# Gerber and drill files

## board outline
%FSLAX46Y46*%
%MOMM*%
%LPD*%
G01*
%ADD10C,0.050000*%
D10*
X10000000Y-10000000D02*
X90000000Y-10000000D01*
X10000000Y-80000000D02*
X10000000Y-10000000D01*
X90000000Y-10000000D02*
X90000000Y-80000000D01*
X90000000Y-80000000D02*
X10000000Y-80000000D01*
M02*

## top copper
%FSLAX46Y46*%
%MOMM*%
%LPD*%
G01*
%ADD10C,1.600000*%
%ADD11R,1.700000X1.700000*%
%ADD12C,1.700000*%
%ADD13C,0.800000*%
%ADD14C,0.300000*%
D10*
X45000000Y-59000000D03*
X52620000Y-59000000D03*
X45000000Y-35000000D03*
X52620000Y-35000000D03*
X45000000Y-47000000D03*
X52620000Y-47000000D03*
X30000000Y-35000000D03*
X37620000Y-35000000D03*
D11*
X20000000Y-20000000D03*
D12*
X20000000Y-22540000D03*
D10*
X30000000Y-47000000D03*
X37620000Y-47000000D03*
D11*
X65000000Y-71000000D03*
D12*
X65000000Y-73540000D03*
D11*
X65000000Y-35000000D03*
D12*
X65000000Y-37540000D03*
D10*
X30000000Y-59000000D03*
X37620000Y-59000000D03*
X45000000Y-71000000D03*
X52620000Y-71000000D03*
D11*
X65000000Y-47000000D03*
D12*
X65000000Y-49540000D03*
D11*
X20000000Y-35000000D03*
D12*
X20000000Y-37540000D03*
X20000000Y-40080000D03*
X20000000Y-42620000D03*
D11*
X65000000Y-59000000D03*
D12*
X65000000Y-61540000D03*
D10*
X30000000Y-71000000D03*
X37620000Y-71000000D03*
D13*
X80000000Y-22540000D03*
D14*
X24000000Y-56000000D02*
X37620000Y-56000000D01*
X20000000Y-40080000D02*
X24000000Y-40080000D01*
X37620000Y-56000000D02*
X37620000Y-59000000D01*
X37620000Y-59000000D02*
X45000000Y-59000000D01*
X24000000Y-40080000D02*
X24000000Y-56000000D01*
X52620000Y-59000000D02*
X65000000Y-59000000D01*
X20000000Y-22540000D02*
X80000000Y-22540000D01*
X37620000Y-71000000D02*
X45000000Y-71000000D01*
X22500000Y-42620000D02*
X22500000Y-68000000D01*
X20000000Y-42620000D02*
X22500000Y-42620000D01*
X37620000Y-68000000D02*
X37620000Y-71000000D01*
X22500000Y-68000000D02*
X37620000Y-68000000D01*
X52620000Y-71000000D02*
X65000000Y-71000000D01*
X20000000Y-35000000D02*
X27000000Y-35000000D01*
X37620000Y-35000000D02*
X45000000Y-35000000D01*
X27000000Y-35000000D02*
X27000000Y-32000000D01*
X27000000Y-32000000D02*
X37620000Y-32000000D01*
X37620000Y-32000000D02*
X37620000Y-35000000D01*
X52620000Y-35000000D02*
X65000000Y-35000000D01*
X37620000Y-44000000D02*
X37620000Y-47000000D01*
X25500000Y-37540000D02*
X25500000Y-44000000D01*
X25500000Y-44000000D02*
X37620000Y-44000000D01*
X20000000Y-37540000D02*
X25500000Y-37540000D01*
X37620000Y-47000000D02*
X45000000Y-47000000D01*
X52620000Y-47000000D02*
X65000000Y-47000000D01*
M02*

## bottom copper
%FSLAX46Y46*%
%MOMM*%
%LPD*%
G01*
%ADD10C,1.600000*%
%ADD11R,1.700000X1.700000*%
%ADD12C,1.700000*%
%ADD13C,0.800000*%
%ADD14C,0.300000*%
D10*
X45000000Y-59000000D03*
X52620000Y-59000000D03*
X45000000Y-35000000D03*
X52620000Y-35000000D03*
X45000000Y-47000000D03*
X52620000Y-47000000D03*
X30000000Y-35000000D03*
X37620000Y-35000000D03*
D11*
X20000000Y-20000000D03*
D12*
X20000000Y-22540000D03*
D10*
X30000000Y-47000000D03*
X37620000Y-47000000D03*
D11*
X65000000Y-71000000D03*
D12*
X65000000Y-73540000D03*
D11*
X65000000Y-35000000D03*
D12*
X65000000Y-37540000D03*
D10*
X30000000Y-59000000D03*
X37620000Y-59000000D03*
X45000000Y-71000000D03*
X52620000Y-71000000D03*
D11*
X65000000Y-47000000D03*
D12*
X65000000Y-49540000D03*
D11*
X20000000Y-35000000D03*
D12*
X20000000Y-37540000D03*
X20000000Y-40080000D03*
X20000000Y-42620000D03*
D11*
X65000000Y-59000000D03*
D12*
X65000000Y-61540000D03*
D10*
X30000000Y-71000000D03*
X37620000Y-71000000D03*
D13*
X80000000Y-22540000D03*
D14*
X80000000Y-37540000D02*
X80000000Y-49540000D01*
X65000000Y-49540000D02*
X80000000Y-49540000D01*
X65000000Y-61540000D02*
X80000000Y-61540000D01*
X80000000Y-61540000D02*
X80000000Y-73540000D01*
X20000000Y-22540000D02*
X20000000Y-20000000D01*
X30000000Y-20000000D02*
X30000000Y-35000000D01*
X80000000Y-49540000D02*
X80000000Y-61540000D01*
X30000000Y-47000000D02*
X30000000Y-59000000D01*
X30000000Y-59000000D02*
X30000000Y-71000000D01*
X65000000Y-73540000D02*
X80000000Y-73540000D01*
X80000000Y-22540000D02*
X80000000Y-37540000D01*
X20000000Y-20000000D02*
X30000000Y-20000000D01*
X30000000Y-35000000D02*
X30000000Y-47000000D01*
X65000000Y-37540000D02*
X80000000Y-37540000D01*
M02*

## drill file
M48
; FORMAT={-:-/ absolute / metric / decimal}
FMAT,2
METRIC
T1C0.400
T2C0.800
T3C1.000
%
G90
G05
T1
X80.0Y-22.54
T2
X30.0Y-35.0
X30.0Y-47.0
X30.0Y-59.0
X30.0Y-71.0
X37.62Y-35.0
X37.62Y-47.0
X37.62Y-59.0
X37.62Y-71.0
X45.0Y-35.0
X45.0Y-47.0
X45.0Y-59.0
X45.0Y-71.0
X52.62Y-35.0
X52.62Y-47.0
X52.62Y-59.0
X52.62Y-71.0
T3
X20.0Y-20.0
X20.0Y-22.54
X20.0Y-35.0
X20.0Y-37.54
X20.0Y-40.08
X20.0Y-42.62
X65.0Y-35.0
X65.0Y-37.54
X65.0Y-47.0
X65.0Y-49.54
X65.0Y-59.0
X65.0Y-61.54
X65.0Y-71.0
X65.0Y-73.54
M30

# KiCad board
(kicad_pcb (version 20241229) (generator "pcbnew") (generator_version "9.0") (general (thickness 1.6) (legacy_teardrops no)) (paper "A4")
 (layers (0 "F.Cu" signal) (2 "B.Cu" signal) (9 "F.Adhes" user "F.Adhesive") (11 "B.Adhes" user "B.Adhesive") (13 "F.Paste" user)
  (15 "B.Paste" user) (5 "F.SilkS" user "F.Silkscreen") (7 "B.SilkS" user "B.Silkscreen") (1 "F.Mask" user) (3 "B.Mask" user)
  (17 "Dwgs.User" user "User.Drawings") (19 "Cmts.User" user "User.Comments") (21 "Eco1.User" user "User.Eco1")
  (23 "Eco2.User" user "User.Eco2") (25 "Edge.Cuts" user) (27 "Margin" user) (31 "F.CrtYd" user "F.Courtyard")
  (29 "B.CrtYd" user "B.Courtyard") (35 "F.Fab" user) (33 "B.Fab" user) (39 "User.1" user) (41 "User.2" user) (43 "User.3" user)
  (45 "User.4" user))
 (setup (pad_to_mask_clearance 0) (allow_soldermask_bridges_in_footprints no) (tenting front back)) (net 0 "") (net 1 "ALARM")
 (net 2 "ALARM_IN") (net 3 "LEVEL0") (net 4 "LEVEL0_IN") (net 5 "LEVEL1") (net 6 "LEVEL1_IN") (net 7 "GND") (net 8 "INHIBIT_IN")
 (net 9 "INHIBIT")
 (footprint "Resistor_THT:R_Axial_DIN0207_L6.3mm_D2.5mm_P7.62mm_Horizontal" (layer "F.Cu") (at 45 59)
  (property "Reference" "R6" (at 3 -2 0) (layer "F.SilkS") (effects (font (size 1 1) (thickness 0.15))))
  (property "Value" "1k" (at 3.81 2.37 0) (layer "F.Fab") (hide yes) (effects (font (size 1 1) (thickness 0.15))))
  (pad "1" thru_hole circle (at 0 0) (size 1.6 1.6) (drill 0.8) (layers "*.Cu" "*.Mask") (remove_unused_layers no) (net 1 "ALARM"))
  (pad "2" thru_hole circle (at 7.62 0) (size 1.6 1.6) (drill 0.8) (layers "*.Cu" "*.Mask") (remove_unused_layers no) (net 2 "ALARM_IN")))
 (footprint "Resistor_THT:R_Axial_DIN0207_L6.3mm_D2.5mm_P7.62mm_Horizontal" (layer "F.Cu") (at 45 35)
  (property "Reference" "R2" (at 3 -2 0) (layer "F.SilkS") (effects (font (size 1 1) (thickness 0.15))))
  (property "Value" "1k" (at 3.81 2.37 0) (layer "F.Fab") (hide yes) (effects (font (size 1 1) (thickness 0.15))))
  (pad "1" thru_hole circle (at 0 0) (size 1.6 1.6) (drill 0.8) (layers "*.Cu" "*.Mask") (remove_unused_layers no) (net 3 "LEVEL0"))
  (pad "2" thru_hole circle (at 7.62 0) (size 1.6 1.6) (drill 0.8) (layers "*.Cu" "*.Mask") (remove_unused_layers no) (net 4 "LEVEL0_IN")))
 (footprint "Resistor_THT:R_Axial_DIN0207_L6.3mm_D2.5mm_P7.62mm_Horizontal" (layer "F.Cu") (at 45 47)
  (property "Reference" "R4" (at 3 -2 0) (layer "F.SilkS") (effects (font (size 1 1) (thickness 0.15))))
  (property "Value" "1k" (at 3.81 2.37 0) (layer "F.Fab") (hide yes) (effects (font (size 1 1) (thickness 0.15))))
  (pad "1" thru_hole circle (at 0 0) (size 1.6 1.6) (drill 0.8) (layers "*.Cu" "*.Mask") (remove_unused_layers no) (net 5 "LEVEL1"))
  (pad "2" thru_hole circle (at 7.62 0) (size 1.6 1.6) (drill 0.8) (layers "*.Cu" "*.Mask") (remove_unused_layers no) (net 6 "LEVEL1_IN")))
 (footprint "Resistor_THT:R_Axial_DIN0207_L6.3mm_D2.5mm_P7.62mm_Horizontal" (layer "F.Cu") (at 30 35)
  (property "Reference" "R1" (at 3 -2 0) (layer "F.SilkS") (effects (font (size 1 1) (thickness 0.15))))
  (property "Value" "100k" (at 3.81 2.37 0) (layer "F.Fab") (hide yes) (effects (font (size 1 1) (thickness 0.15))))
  (pad "1" thru_hole circle (at 0 0) (size 1.6 1.6) (drill 0.8) (layers "*.Cu" "*.Mask") (remove_unused_layers no) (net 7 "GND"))
  (pad "2" thru_hole circle (at 7.62 0) (size 1.6 1.6) (drill 0.8) (layers "*.Cu" "*.Mask") (remove_unused_layers no) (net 3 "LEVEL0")))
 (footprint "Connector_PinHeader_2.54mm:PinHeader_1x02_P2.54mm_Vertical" (layer "F.Cu") (at 20 20)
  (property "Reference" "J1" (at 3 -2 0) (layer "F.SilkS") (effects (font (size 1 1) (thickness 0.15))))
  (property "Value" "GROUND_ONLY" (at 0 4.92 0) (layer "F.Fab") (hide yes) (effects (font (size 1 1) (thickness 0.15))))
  (pad "1" thru_hole rect (at 0 0) (size 1.7 1.7) (drill 1) (layers "*.Cu" "*.Mask") (remove_unused_layers no) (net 7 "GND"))
  (pad "2" thru_hole circle (at 0 2.54) (size 1.7 1.7) (drill 1) (layers "*.Cu" "*.Mask") (remove_unused_layers no) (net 7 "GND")))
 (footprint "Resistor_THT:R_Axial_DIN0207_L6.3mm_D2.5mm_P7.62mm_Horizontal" (layer "F.Cu") (at 30 47)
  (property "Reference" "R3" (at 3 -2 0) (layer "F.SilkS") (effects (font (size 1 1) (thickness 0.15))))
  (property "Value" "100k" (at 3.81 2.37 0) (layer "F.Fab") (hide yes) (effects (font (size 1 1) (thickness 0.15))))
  (pad "1" thru_hole circle (at 0 0) (size 1.6 1.6) (drill 0.8) (layers "*.Cu" "*.Mask") (remove_unused_layers no) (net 7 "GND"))
  (pad "2" thru_hole circle (at 7.62 0) (size 1.6 1.6) (drill 0.8) (layers "*.Cu" "*.Mask") (remove_unused_layers no) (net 5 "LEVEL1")))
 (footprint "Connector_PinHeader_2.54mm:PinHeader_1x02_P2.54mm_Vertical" (layer "F.Cu") (at 65 71)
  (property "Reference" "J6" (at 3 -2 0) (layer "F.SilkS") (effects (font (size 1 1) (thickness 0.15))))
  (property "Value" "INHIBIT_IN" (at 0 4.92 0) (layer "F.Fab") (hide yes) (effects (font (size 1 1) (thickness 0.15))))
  (pad "1" thru_hole rect (at 0 0) (size 1.7 1.7) (drill 1) (layers "*.Cu" "*.Mask") (remove_unused_layers no) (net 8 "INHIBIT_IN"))
  (pad "2" thru_hole circle (at 0 2.54) (size 1.7 1.7) (drill 1) (layers "*.Cu" "*.Mask") (remove_unused_layers no) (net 7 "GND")))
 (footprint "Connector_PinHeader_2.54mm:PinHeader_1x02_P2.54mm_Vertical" (layer "F.Cu") (at 65 35)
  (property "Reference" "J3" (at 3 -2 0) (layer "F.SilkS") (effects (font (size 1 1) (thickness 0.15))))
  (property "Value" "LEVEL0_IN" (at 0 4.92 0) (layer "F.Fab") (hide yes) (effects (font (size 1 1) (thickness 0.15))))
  (pad "1" thru_hole rect (at 0 0) (size 1.7 1.7) (drill 1) (layers "*.Cu" "*.Mask") (remove_unused_layers no) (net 4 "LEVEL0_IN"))
  (pad "2" thru_hole circle (at 0 2.54) (size 1.7 1.7) (drill 1) (layers "*.Cu" "*.Mask") (remove_unused_layers no) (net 7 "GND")))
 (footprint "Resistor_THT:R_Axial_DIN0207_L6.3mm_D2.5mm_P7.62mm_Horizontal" (layer "F.Cu") (at 30 59)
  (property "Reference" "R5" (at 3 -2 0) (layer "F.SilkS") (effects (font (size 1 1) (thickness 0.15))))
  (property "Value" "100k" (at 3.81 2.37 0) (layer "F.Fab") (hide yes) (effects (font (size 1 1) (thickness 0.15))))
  (pad "1" thru_hole circle (at 0 0) (size 1.6 1.6) (drill 0.8) (layers "*.Cu" "*.Mask") (remove_unused_layers no) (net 7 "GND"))
  (pad "2" thru_hole circle (at 7.62 0) (size 1.6 1.6) (drill 0.8) (layers "*.Cu" "*.Mask") (remove_unused_layers no) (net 1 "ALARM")))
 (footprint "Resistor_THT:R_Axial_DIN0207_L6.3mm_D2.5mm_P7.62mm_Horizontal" (layer "F.Cu") (at 45 71)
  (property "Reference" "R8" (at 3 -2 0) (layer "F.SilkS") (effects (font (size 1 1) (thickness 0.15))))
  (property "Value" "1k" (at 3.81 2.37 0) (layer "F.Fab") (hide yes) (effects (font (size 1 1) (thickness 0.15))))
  (pad "1" thru_hole circle (at 0 0) (size 1.6 1.6) (drill 0.8) (layers "*.Cu" "*.Mask") (remove_unused_layers no) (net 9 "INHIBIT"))
  (pad "2" thru_hole circle (at 7.62 0) (size 1.6 1.6) (drill 0.8) (layers "*.Cu" "*.Mask") (remove_unused_layers no) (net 8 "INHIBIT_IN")))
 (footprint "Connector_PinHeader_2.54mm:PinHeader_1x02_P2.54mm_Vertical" (layer "F.Cu") (at 65 47)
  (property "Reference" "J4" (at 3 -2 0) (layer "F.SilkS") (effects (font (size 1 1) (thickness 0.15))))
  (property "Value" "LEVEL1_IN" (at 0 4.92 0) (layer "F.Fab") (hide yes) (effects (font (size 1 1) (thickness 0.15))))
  (pad "1" thru_hole rect (at 0 0) (size 1.7 1.7) (drill 1) (layers "*.Cu" "*.Mask") (remove_unused_layers no) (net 6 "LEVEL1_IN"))
  (pad "2" thru_hole circle (at 0 2.54) (size 1.7 1.7) (drill 1) (layers "*.Cu" "*.Mask") (remove_unused_layers no) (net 7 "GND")))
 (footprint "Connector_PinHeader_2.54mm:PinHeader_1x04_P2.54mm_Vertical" (layer "F.Cu") (at 20 35)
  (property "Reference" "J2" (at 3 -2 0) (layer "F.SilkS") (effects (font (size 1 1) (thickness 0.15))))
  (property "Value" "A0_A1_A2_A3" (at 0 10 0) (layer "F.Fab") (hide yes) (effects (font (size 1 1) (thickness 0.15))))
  (pad "1" thru_hole rect (at 0 0) (size 1.7 1.7) (drill 1) (layers "*.Cu" "*.Mask") (remove_unused_layers no) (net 3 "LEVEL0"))
  (pad "2" thru_hole circle (at 0 2.54) (size 1.7 1.7) (drill 1) (layers "*.Cu" "*.Mask") (remove_unused_layers no) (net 5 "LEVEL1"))
  (pad "3" thru_hole circle (at 0 5.08) (size 1.7 1.7) (drill 1) (layers "*.Cu" "*.Mask") (remove_unused_layers no) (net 1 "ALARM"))
  (pad "4" thru_hole circle (at 0 7.62) (size 1.7 1.7) (drill 1) (layers "*.Cu" "*.Mask") (remove_unused_layers no) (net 9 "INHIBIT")))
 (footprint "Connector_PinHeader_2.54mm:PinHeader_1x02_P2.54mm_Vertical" (layer "F.Cu") (at 65 59)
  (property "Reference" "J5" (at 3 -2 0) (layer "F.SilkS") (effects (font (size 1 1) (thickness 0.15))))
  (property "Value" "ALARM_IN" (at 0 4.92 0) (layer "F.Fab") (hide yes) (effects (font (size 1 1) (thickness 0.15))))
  (pad "1" thru_hole rect (at 0 0) (size 1.7 1.7) (drill 1) (layers "*.Cu" "*.Mask") (remove_unused_layers no) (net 2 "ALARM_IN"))
  (pad "2" thru_hole circle (at 0 2.54) (size 1.7 1.7) (drill 1) (layers "*.Cu" "*.Mask") (remove_unused_layers no) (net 7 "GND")))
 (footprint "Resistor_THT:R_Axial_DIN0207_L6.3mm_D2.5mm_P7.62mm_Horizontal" (layer "F.Cu") (at 30 71)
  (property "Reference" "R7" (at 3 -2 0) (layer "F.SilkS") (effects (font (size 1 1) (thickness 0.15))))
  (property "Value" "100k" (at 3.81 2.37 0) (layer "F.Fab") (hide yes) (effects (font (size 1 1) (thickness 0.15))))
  (pad "1" thru_hole circle (at 0 0) (size 1.6 1.6) (drill 0.8) (layers "*.Cu" "*.Mask") (remove_unused_layers no) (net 7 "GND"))
  (pad "2" thru_hole circle (at 7.62 0) (size 1.6 1.6) (drill 0.8) (layers "*.Cu" "*.Mask") (remove_unused_layers no) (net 9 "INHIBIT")))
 (gr_line (start 10 10) (end 90 10) (stroke (width 0.05) (type default)) (layer "Edge.Cuts"))
 (gr_line (start 10 80) (end 10 10) (stroke (width 0.05) (type default)) (layer "Edge.Cuts"))
 (gr_line (start 90 10) (end 90 80) (stroke (width 0.05) (type default)) (layer "Edge.Cuts"))
 (gr_line (start 90 80) (end 10 80) (stroke (width 0.05) (type default)) (layer "Edge.Cuts"))
 (segment (start 24 56) (end 37.62 56) (width 0.3) (layer "F.Cu") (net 1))
 (segment (start 20 40.08) (end 24 40.08) (width 0.3) (layer "F.Cu") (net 1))
 (segment (start 37.62 56) (end 37.62 59) (width 0.3) (layer "F.Cu") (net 1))
 (segment (start 37.62 59) (end 45 59) (width 0.3) (layer "F.Cu") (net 1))
 (segment (start 24 40.08) (end 24 56) (width 0.3) (layer "F.Cu") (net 1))
 (segment (start 52.62 59) (end 65 59) (width 0.3) (layer "F.Cu") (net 2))
 (segment (start 20 22.54) (end 80 22.54) (width 0.3) (layer "F.Cu") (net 7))
 (via (at 80 22.54) (size 0.8) (drill 0.4) (layers "F.Cu" "B.Cu") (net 7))
 (segment (start 80 37.54) (end 80 49.54) (width 0.3) (layer "B.Cu") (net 7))
 (segment (start 65 49.54) (end 80 49.54) (width 0.3) (layer "B.Cu") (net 7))
 (segment (start 65 61.54) (end 80 61.54) (width 0.3) (layer "B.Cu") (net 7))
 (segment (start 80 61.54) (end 80 73.54) (width 0.3) (layer "B.Cu") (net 7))
 (segment (start 20 22.54) (end 20 20) (width 0.3) (layer "B.Cu") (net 7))
 (segment (start 30 20) (end 30 35) (width 0.3) (layer "B.Cu") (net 7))
 (segment (start 80 49.54) (end 80 61.54) (width 0.3) (layer "B.Cu") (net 7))
 (segment (start 30 47) (end 30 59) (width 0.3) (layer "B.Cu") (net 7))
 (segment (start 30 59) (end 30 71) (width 0.3) (layer "B.Cu") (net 7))
 (segment (start 65 73.54) (end 80 73.54) (width 0.3) (layer "B.Cu") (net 7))
 (segment (start 80 22.54) (end 80 37.54) (width 0.3) (layer "B.Cu") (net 7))
 (segment (start 20 20) (end 30 20) (width 0.3) (layer "B.Cu") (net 7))
 (segment (start 30 35) (end 30 47) (width 0.3) (layer "B.Cu") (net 7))
 (segment (start 65 37.54) (end 80 37.54) (width 0.3) (layer "B.Cu") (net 7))
 (segment (start 37.62 71) (end 45 71) (width 0.3) (layer "F.Cu") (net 9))
 (segment (start 22.5 42.62) (end 22.5 68) (width 0.3) (layer "F.Cu") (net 9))
 (segment (start 20 42.62) (end 22.5 42.62) (width 0.3) (layer "F.Cu") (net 9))
 (segment (start 37.62 68) (end 37.62 71) (width 0.3) (layer "F.Cu") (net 9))
 (segment (start 22.5 68) (end 37.62 68) (width 0.3) (layer "F.Cu") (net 9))
 (segment (start 52.62 71) (end 65 71) (width 0.3) (layer "F.Cu") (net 8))
 (segment (start 20 35) (end 27 35) (width 0.3) (layer "F.Cu") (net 3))
 (segment (start 37.62 35) (end 45 35) (width 0.3) (layer "F.Cu") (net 3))
 (segment (start 27 35) (end 27 32) (width 0.3) (layer "F.Cu") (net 3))
 (segment (start 27 32) (end 37.62 32) (width 0.3) (layer "F.Cu") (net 3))
 (segment (start 37.62 32) (end 37.62 35) (width 0.3) (layer "F.Cu") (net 3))
 (segment (start 52.62 35) (end 65 35) (width 0.3) (layer "F.Cu") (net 4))
 (segment (start 37.62 44) (end 37.62 47) (width 0.3) (layer "F.Cu") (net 5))
 (segment (start 25.5 37.54) (end 25.5 44) (width 0.3) (layer "F.Cu") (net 5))
 (segment (start 25.5 44) (end 37.62 44) (width 0.3) (layer "F.Cu") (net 5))
 (segment (start 20 37.54) (end 25.5 37.54) (width 0.3) (layer "F.Cu") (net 5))
 (segment (start 37.62 47) (end 45 47) (width 0.3) (layer "F.Cu") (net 5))
 (segment (start 52.62 47) (end 65 47) (width 0.3) (layer "F.Cu") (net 6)))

